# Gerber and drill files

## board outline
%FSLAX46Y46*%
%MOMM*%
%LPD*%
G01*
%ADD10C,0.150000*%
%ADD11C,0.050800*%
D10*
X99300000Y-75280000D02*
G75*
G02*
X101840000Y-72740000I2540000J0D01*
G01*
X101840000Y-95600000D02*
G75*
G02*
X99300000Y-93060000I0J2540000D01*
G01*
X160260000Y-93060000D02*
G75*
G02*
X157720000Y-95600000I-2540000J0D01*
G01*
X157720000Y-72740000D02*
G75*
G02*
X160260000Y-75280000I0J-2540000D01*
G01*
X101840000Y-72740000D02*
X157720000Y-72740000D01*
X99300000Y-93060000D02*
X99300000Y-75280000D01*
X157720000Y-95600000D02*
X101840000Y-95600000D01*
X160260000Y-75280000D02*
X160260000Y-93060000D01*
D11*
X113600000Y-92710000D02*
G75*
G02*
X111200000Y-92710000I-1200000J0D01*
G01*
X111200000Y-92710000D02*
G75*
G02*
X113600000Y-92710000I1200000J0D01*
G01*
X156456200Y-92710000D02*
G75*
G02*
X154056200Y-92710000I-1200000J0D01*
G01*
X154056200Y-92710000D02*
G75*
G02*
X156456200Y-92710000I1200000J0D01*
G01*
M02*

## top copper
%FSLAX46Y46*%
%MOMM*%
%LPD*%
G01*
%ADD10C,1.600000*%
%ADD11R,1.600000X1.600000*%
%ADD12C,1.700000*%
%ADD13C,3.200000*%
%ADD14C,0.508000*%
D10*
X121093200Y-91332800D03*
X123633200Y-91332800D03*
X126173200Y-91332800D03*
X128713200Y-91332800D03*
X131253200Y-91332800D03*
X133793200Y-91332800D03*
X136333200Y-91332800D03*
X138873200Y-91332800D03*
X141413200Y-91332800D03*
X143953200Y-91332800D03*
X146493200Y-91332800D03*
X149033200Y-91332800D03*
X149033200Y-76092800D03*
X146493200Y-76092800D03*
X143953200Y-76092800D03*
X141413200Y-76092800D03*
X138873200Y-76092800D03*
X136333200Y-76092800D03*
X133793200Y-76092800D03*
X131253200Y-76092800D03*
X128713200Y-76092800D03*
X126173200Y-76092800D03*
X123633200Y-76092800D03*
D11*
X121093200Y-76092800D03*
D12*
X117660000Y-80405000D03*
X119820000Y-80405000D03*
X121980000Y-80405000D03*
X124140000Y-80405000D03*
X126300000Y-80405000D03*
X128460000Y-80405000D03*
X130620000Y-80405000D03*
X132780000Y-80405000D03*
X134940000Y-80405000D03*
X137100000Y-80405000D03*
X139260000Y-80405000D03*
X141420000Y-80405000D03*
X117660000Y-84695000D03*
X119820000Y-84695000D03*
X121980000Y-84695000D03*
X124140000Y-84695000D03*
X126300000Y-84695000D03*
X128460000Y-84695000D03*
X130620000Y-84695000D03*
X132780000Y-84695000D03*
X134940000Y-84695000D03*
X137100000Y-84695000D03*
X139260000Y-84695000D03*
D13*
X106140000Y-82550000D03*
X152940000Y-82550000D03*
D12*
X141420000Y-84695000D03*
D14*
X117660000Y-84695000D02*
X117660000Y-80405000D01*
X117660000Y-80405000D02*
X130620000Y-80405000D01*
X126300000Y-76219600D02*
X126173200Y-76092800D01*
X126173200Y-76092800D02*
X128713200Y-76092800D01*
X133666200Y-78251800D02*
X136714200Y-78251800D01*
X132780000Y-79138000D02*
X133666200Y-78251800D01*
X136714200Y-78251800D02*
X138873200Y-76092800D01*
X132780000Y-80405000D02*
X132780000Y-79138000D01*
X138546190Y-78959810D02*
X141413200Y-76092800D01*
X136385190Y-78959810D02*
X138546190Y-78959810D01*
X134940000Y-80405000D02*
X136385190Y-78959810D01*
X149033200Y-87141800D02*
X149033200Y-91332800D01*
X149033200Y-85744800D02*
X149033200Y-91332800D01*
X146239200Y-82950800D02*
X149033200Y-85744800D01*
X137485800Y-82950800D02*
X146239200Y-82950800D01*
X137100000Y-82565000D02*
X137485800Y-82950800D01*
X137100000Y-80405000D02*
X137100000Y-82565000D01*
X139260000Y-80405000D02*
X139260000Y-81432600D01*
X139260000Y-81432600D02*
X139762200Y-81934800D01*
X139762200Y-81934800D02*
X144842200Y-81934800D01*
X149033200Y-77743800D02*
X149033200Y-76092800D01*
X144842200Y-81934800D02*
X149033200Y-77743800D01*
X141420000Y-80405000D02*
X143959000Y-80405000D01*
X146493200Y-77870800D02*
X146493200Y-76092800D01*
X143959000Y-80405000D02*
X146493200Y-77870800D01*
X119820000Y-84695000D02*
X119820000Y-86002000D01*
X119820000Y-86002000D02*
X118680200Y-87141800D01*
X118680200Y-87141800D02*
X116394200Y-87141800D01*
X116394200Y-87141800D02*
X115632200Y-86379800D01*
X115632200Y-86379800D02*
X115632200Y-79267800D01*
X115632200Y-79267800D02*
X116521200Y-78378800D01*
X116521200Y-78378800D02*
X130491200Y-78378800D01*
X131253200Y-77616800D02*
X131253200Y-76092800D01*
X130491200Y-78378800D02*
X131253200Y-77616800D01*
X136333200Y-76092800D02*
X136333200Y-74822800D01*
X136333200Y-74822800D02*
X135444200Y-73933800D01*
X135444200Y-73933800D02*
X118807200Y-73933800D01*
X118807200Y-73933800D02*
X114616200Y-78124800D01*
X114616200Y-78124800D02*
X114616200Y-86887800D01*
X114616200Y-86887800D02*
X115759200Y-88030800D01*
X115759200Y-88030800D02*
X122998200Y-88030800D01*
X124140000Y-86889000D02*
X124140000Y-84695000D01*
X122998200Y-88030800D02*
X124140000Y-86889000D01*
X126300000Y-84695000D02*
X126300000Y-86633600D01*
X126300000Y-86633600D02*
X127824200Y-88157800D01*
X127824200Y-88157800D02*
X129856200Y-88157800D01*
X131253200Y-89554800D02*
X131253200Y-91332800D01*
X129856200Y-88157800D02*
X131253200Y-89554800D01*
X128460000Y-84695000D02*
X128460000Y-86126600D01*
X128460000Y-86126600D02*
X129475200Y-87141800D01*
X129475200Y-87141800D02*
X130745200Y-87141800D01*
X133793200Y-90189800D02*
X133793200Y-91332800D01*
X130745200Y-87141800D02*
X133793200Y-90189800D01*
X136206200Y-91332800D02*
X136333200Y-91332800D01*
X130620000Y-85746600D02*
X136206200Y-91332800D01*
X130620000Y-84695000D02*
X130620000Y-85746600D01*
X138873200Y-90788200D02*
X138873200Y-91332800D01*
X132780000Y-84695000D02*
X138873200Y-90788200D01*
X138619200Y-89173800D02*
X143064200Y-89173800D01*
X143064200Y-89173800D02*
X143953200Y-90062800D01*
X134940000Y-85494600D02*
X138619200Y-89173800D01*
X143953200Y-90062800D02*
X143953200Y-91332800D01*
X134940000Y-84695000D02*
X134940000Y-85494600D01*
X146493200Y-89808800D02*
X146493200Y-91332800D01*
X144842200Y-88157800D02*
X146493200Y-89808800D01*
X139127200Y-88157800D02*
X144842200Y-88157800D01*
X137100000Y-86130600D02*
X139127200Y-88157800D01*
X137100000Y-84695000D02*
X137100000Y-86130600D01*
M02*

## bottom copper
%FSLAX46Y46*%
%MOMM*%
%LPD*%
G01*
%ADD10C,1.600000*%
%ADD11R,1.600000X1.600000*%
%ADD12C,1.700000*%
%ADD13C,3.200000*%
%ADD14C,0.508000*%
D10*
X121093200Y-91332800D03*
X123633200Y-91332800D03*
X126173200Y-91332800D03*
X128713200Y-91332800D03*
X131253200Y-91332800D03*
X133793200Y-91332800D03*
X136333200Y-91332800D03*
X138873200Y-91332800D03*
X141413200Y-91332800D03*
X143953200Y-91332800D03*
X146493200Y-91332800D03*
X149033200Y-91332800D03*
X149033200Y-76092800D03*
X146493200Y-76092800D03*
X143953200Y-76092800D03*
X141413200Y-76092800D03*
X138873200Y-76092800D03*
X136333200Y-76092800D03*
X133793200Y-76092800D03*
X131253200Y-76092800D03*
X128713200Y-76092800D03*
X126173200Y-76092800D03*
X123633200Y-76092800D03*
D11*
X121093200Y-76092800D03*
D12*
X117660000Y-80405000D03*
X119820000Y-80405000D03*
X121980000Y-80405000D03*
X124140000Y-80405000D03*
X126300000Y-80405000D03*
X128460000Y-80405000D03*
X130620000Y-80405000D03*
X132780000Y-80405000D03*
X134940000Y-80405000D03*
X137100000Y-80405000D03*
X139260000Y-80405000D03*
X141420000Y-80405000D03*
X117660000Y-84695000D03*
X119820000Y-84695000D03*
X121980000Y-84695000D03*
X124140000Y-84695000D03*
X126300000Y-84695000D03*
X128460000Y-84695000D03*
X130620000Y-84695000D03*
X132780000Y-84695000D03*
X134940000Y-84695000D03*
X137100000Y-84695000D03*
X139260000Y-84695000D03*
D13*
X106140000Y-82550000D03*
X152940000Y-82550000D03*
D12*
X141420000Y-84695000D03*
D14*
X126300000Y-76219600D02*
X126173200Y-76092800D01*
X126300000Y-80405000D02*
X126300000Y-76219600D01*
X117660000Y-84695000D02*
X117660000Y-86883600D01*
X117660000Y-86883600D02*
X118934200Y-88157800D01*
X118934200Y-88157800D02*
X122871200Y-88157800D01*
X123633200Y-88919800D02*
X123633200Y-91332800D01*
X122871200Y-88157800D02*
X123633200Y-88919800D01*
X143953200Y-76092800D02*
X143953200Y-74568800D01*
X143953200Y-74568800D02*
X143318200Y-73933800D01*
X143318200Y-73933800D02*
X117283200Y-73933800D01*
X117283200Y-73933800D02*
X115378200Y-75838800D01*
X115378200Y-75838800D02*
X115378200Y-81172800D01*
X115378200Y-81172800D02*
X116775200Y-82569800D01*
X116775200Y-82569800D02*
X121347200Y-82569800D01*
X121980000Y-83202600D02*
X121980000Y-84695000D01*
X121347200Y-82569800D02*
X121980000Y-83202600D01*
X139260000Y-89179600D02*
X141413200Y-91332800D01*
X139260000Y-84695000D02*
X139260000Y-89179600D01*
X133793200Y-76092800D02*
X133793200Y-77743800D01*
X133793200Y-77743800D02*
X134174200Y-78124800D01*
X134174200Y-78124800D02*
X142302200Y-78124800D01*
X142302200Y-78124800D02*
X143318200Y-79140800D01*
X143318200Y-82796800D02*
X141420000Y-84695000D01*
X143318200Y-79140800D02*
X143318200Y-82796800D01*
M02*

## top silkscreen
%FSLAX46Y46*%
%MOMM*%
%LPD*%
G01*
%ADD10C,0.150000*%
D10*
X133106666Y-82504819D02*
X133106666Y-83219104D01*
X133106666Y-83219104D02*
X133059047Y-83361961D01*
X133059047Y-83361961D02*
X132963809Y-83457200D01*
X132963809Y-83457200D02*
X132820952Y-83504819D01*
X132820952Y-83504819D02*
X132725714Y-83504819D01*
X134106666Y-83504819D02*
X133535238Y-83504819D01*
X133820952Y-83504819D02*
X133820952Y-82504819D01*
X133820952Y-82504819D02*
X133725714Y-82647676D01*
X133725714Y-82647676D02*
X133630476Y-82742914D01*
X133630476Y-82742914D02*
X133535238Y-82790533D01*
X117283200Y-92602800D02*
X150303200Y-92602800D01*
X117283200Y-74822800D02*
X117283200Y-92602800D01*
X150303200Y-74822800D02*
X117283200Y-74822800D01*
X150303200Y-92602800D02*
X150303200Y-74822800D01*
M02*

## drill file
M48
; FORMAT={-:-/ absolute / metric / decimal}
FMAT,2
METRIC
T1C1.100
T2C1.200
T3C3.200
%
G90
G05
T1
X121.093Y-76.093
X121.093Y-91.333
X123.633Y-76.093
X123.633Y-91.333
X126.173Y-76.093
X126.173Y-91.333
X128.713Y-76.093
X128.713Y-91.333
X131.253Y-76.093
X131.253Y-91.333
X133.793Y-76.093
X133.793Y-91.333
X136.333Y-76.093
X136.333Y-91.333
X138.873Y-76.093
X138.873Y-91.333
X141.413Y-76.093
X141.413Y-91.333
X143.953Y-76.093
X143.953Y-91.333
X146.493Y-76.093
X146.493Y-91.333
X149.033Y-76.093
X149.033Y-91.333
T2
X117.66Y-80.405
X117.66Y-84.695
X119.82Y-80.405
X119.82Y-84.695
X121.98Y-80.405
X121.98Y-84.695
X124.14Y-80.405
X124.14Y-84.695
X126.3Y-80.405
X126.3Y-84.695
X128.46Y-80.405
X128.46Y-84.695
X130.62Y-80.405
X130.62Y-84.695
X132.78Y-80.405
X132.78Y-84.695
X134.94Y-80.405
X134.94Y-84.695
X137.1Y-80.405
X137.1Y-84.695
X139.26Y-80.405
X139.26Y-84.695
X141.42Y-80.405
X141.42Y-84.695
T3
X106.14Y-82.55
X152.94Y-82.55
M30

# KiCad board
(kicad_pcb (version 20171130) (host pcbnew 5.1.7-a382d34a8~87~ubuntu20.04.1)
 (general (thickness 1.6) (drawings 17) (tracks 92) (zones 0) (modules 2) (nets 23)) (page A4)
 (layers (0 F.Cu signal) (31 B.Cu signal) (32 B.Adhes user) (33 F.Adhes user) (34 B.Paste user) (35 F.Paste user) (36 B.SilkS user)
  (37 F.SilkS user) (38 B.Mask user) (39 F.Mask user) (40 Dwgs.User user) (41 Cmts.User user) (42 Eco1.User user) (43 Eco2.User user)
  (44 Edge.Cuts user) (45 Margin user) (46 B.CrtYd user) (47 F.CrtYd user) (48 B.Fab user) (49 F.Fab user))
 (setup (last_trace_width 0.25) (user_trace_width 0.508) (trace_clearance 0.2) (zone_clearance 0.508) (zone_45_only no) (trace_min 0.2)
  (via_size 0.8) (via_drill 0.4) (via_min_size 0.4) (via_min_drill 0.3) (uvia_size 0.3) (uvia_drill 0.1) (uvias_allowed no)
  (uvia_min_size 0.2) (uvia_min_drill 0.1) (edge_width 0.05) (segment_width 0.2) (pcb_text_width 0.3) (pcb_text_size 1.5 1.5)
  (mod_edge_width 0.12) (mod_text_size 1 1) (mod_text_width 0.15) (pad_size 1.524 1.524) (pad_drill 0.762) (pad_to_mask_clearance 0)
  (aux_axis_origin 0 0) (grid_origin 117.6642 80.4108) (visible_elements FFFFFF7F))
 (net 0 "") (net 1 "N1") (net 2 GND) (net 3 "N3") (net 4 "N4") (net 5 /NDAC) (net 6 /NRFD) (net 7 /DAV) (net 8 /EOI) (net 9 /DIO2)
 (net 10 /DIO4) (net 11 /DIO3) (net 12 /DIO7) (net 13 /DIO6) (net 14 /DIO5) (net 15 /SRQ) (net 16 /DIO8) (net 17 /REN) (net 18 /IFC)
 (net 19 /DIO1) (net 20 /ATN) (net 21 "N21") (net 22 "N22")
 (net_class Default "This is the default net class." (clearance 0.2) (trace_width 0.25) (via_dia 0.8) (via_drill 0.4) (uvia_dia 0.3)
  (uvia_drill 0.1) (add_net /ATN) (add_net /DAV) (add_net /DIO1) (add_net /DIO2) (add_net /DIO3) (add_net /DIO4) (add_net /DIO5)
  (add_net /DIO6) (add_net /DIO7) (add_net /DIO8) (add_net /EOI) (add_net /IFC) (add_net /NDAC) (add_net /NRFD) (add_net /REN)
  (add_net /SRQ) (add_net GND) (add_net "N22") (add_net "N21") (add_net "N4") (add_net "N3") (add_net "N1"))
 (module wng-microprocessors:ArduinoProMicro (layer B.Cu) (at 135.0632 83.7128)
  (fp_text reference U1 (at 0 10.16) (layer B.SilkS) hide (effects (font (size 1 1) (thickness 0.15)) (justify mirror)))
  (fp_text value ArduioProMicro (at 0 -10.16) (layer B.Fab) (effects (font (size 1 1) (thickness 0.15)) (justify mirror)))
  (fp_line (start -17.78 8.89) (end 15.24 8.89) (layer F.SilkS) (width 0.15))
  (fp_line (start -17.78 -8.89) (end -17.78 8.89) (layer F.SilkS) (width 0.15))
  (fp_line (start 15.24 -8.89) (end -17.78 -8.89) (layer F.SilkS) (width 0.15))
  (fp_line (start 15.24 8.89) (end 15.24 -8.89) (layer F.SilkS) (width 0.15))
  (pad 24 thru_hole circle (at -13.97 7.62) (size 1.6 1.6) (drill 1.1) (layers *.Cu *.Mask B.SilkS) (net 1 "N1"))
  (pad 23 thru_hole circle (at -11.43 7.62) (size 1.6 1.6) (drill 1.1) (layers *.Cu *.Mask B.SilkS) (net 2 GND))
  (pad 22 thru_hole circle (at -8.89 7.62) (size 1.6 1.6) (drill 1.1) (layers *.Cu *.Mask B.SilkS) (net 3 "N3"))
  (pad 21 thru_hole circle (at -6.35 7.62) (size 1.6 1.6) (drill 1.1) (layers *.Cu *.Mask B.SilkS) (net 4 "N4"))
  (pad 20 thru_hole circle (at -3.81 7.62) (size 1.6 1.6) (drill 1.1) (layers *.Cu *.Mask B.SilkS) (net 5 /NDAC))
  (pad 19 thru_hole circle (at -1.27 7.62) (size 1.6 1.6) (drill 1.1) (layers *.Cu *.Mask B.SilkS) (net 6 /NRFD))
  (pad 18 thru_hole circle (at 1.27 7.62) (size 1.6 1.6) (drill 1.1) (layers *.Cu *.Mask B.SilkS) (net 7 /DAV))
  (pad 17 thru_hole circle (at 3.81 7.62) (size 1.6 1.6) (drill 1.1) (layers *.Cu *.Mask B.SilkS) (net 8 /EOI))
  (pad 16 thru_hole circle (at 6.35 7.62) (size 1.6 1.6) (drill 1.1) (layers *.Cu *.Mask B.SilkS) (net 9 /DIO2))
  (pad 15 thru_hole circle (at 8.89 7.62) (size 1.6 1.6) (drill 1.1) (layers *.Cu *.Mask B.SilkS) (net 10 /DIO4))
  (pad 14 thru_hole circle (at 11.43 7.62) (size 1.6 1.6) (drill 1.1) (layers *.Cu *.Mask B.SilkS) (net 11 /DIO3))
  (pad 13 thru_hole circle (at 13.97 7.62) (size 1.6 1.6) (drill 1.1) (layers *.Cu *.Mask B.SilkS) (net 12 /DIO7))
  (pad 12 thru_hole circle (at 13.97 -7.62) (size 1.6 1.6) (drill 1.1) (layers *.Cu *.Mask B.SilkS) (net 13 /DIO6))
  (pad 11 thru_hole circle (at 11.43 -7.62) (size 1.6 1.6) (drill 1.1) (layers *.Cu *.Mask B.SilkS) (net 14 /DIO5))
  (pad 10 thru_hole circle (at 8.89 -7.62) (size 1.6 1.6) (drill 1.1) (layers *.Cu *.Mask B.SilkS) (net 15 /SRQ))
  (pad 9 thru_hole circle (at 6.35 -7.62) (size 1.6 1.6) (drill 1.1) (layers *.Cu *.Mask B.SilkS) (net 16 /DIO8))
  (pad 8 thru_hole circle (at 3.81 -7.62) (size 1.6 1.6) (drill 1.1) (layers *.Cu *.Mask B.SilkS) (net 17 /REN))
  (pad 7 thru_hole circle (at 1.27 -7.62) (size 1.6 1.6) (drill 1.1) (layers *.Cu *.Mask B.SilkS) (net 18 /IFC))
  (pad 6 thru_hole circle (at -1.27 -7.62) (size 1.6 1.6) (drill 1.1) (layers *.Cu *.Mask B.SilkS) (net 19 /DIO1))
  (pad 5 thru_hole circle (at -3.81 -7.62) (size 1.6 1.6) (drill 1.1) (layers *.Cu *.Mask B.SilkS) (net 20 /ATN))
  (pad 4 thru_hole circle (at -6.35 -7.62) (size 1.6 1.6) (drill 1.1) (layers *.Cu *.Mask B.SilkS) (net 2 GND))
  (pad 3 thru_hole circle (at -8.89 -7.62) (size 1.6 1.6) (drill 1.1) (layers *.Cu *.Mask B.SilkS) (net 2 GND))
  (pad 2 thru_hole circle (at -11.43 -7.62) (size 1.6 1.6) (drill 1.1) (layers *.Cu *.Mask B.SilkS) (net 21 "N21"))
  (pad 1 thru_hole rect (at -13.97 -7.62) (size 1.6 1.6) (drill 1.1) (layers *.Cu *.Mask B.SilkS) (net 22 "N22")))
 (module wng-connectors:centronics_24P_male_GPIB (layer F.Cu) (at 129.54 82.55)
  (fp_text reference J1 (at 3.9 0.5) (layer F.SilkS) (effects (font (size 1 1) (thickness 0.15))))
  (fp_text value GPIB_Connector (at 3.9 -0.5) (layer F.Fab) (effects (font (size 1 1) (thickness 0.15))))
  (pad 24 thru_hole circle (at -11.88 -2.145) (size 1.7 1.7) (drill 1.2) (layers *.Cu *.Mask) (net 2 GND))
  (pad 23 thru_hole circle (at -9.72 -2.145) (size 1.7 1.7) (drill 1.2) (layers *.Cu *.Mask) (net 2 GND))
  (pad 22 thru_hole circle (at -7.56 -2.145) (size 1.7 1.7) (drill 1.2) (layers *.Cu *.Mask) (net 2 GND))
  (pad 21 thru_hole circle (at -5.4 -2.145) (size 1.7 1.7) (drill 1.2) (layers *.Cu *.Mask) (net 2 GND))
  (pad 20 thru_hole circle (at -3.24 -2.145) (size 1.7 1.7) (drill 1.2) (layers *.Cu *.Mask) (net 2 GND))
  (pad 19 thru_hole circle (at -1.08 -2.145) (size 1.7 1.7) (drill 1.2) (layers *.Cu *.Mask) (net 2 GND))
  (pad 18 thru_hole circle (at 1.08 -2.145) (size 1.7 1.7) (drill 1.2) (layers *.Cu *.Mask) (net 2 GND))
  (pad 17 thru_hole circle (at 3.24 -2.145) (size 1.7 1.7) (drill 1.2) (layers *.Cu *.Mask) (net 17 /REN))
  (pad 16 thru_hole circle (at 5.4 -2.145) (size 1.7 1.7) (drill 1.2) (layers *.Cu *.Mask) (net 16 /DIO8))
  (pad 15 thru_hole circle (at 7.56 -2.145) (size 1.7 1.7) (drill 1.2) (layers *.Cu *.Mask) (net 12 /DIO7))
  (pad 14 thru_hole circle (at 9.72 -2.145) (size 1.7 1.7) (drill 1.2) (layers *.Cu *.Mask) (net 13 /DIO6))
  (pad 13 thru_hole circle (at 11.88 -2.145) (size 1.7 1.7) (drill 1.2) (layers *.Cu *.Mask) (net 14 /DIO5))
  (pad 12 thru_hole circle (at -11.88 2.145) (size 1.7 1.7) (drill 1.2) (layers *.Cu *.Mask) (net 2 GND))
  (pad 11 thru_hole circle (at -9.72 2.145) (size 1.7 1.7) (drill 1.2) (layers *.Cu *.Mask) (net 20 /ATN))
  (pad 10 thru_hole circle (at -7.56 2.145) (size 1.7 1.7) (drill 1.2) (layers *.Cu *.Mask) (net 15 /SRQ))
  (pad 9 thru_hole circle (at -5.4 2.145) (size 1.7 1.7) (drill 1.2) (layers *.Cu *.Mask) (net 18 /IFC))
  (pad 8 thru_hole circle (at -3.24 2.145) (size 1.7 1.7) (drill 1.2) (layers *.Cu *.Mask) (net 5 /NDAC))
  (pad 7 thru_hole circle (at -1.08 2.145) (size 1.7 1.7) (drill 1.2) (layers *.Cu *.Mask) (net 6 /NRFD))
  (pad 6 thru_hole circle (at 1.08 2.145) (size 1.7 1.7) (drill 1.2) (layers *.Cu *.Mask) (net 7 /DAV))
  (pad 5 thru_hole circle (at 3.24 2.145) (size 1.7 1.7) (drill 1.2) (layers *.Cu *.Mask) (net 8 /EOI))
  (pad 4 thru_hole circle (at 5.4 2.145) (size 1.7 1.7) (drill 1.2) (layers *.Cu *.Mask) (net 10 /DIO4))
  (pad 3 thru_hole circle (at 7.56 2.145) (size 1.7 1.7) (drill 1.2) (layers *.Cu *.Mask) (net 11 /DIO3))
  (pad 2 thru_hole circle (at 9.72 2.145) (size 1.7 1.7) (drill 1.2) (layers *.Cu *.Mask) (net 9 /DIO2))
  (pad 26 thru_hole circle (at -23.4 0) (size 3.2 3.2) (drill 3.2) (layers *.Cu *.Mask))
  (pad 25 thru_hole circle (at 23.4 0) (size 3.2 3.2) (drill 3.2) (layers *.Cu *.Mask))
  (pad 1 thru_hole circle (at 11.88 2.145) (size 1.7 1.7) (drill 1.2) (layers *.Cu *.Mask) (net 19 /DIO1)))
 (gr_arc (start 101.84 75.28) (end 101.84 72.74) (angle -90) (layer Edge.Cuts) (width 0.15))
 (gr_arc (start 101.84 93.06) (end 99.3 93.06) (angle -90) (layer Edge.Cuts) (width 0.15))
 (gr_arc (start 157.72 93.06) (end 157.72 95.6) (angle -90) (layer Edge.Cuts) (width 0.15))
 (gr_arc (start 157.72 75.28) (end 160.26 75.28) (angle -90) (layer Edge.Cuts) (width 0.15))
 (gr_line (start 101.84 72.74) (end 157.72 72.74) (layer Edge.Cuts) (width 0.15))
 (gr_line (start 99.3 93.06) (end 99.3 75.28) (layer Edge.Cuts) (width 0.15))
 (gr_line (start 157.72 95.6) (end 101.84 95.6) (layer Edge.Cuts) (width 0.15))
 (gr_line (start 160.26 75.28) (end 160.26 93.06) (layer Edge.Cuts) (width 0.15))
 (gr_circle (center 112.4 92.71) (end 113.6 92.71) (layer Edge.Cuts) (width 0.0508))
 (gr_circle (center 155.2562 92.71) (end 156.4562 92.71) (layer Edge.Cuts) (width 0.0508))
 (segment (start 117.66 84.695) (end 117.66 80.405) (width 0.508) (layer F.Cu) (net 2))
 (segment (start 117.66 80.405) (end 130.62 80.405) (width 0.508) (layer F.Cu) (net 2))
 (segment (start 126.3 76.2196) (end 126.1732 76.0928) (width 0.508) (layer F.Cu) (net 2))
 (segment (start 126.1732 76.0928) (end 128.7132 76.0928) (width 0.508) (layer F.Cu) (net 2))
 (segment (start 126.3 76.2196) (end 126.1732 76.0928) (width 0.508) (layer B.Cu) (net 2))
 (segment (start 126.3 80.405) (end 126.3 76.2196) (width 0.508) (layer B.Cu) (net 2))
 (segment (start 117.66 84.695) (end 117.66 86.8836) (width 0.508) (layer B.Cu) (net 2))
 (segment (start 117.66 86.8836) (end 118.9342 88.1578) (width 0.508) (layer B.Cu) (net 2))
 (segment (start 118.9342 88.1578) (end 122.8712 88.1578) (width 0.508) (layer B.Cu) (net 2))
 (segment (start 123.6332 88.9198) (end 123.6332 91.3328) (width 0.508) (layer B.Cu) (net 2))
 (segment (start 122.8712 88.1578) (end 123.6332 88.9198) (width 0.508) (layer B.Cu) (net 2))
 (segment (start 133.6662 78.2518) (end 136.7142 78.2518) (width 0.508) (layer F.Cu) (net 17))
 (segment (start 132.78 79.138) (end 133.6662 78.2518) (width 0.508) (layer F.Cu) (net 17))
 (segment (start 136.7142 78.2518) (end 138.8732 76.0928) (width 0.508) (layer F.Cu) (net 17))
 (segment (start 132.78 80.405) (end 132.78 79.138) (width 0.508) (layer F.Cu) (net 17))
 (segment (start 138.54619 78.95981) (end 141.4132 76.0928) (width 0.508) (layer F.Cu) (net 16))
 (segment (start 136.38519 78.95981) (end 138.54619 78.95981) (width 0.508) (layer F.Cu) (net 16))
 (segment (start 134.94 80.405) (end 136.38519 78.95981) (width 0.508) (layer F.Cu) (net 16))
 (segment (start 149.0332 87.1418) (end 149.0332 91.3328) (width 0.508) (layer F.Cu) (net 12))
 (segment (start 149.0332 85.7448) (end 149.0332 91.3328) (width 0.508) (layer F.Cu) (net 12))
 (segment (start 146.2392 82.9508) (end 149.0332 85.7448) (width 0.508) (layer F.Cu) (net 12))
 (segment (start 137.4858 82.9508) (end 146.2392 82.9508) (width 0.508) (layer F.Cu) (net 12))
 (segment (start 137.1 82.565) (end 137.4858 82.9508) (width 0.508) (layer F.Cu) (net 12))
 (segment (start 137.1 80.405) (end 137.1 82.565) (width 0.508) (layer F.Cu) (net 12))
 (segment (start 139.26 80.405) (end 139.26 81.4326) (width 0.508) (layer F.Cu) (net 13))
 (segment (start 139.26 81.4326) (end 139.7622 81.9348) (width 0.508) (layer F.Cu) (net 13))
 (segment (start 139.7622 81.9348) (end 144.8422 81.9348) (width 0.508) (layer F.Cu) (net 13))
 (segment (start 149.0332 77.7438) (end 149.0332 76.0928) (width 0.508) (layer F.Cu) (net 13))
 (segment (start 144.8422 81.9348) (end 149.0332 77.7438) (width 0.508) (layer F.Cu) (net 13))
 (segment (start 141.42 80.405) (end 143.959 80.405) (width 0.508) (layer F.Cu) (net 14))
 (segment (start 146.4932 77.8708) (end 146.4932 76.0928) (width 0.508) (layer F.Cu) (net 14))
 (segment (start 143.959 80.405) (end 146.4932 77.8708) (width 0.508) (layer F.Cu) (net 14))
 (segment (start 119.82 84.695) (end 119.82 86.002) (width 0.508) (layer F.Cu) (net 20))
 (segment (start 119.82 86.002) (end 118.6802 87.1418) (width 0.508) (layer F.Cu) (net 20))
 (segment (start 118.6802 87.1418) (end 116.3942 87.1418) (width 0.508) (layer F.Cu) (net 20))
 (segment (start 116.3942 87.1418) (end 115.6322 86.3798) (width 0.508) (layer F.Cu) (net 20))
 (segment (start 115.6322 86.3798) (end 115.6322 79.2678) (width 0.508) (layer F.Cu) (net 20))
 (segment (start 115.6322 79.2678) (end 116.5212 78.3788) (width 0.508) (layer F.Cu) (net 20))
 (segment (start 116.5212 78.3788) (end 130.4912 78.3788) (width 0.508) (layer F.Cu) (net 20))
 (segment (start 131.2532 77.6168) (end 131.2532 76.0928) (width 0.508) (layer F.Cu) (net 20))
 (segment (start 130.4912 78.3788) (end 131.2532 77.6168) (width 0.508) (layer F.Cu) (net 20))
 (segment (start 143.9532 76.0928) (end 143.9532 74.5688) (width 0.508) (layer B.Cu) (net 15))
 (segment (start 143.9532 74.5688) (end 143.3182 73.9338) (width 0.508) (layer B.Cu) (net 15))
 (segment (start 143.3182 73.9338) (end 117.2832 73.9338) (width 0.508) (layer B.Cu) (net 15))
 (segment (start 117.2832 73.9338) (end 115.3782 75.8388) (width 0.508) (layer B.Cu) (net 15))
 (segment (start 115.3782 75.8388) (end 115.3782 81.1728) (width 0.508) (layer B.Cu) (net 15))
 (segment (start 115.3782 81.1728) (end 116.7752 82.5698) (width 0.508) (layer B.Cu) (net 15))
 (segment (start 116.7752 82.5698) (end 121.3472 82.5698) (width 0.508) (layer B.Cu) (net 15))
 (segment (start 121.98 83.2026) (end 121.98 84.695) (width 0.508) (layer B.Cu) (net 15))
 (segment (start 121.3472 82.5698) (end 121.98 83.2026) (width 0.508) (layer B.Cu) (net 15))
 (segment (start 136.3332 76.0928) (end 136.3332 74.8228) (width 0.508) (layer F.Cu) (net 18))
 (segment (start 136.3332 74.8228) (end 135.4442 73.9338) (width 0.508) (layer F.Cu) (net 18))
 (segment (start 135.4442 73.9338) (end 118.8072 73.9338) (width 0.508) (layer F.Cu) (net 18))
 (segment (start 118.8072 73.9338) (end 114.6162 78.1248) (width 0.508) (layer F.Cu) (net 18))
 (segment (start 114.6162 78.1248) (end 114.6162 86.8878) (width 0.508) (layer F.Cu) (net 18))
 (segment (start 114.6162 86.8878) (end 115.7592 88.0308) (width 0.508) (layer F.Cu) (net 18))
 (segment (start 115.7592 88.0308) (end 122.9982 88.0308) (width 0.508) (layer F.Cu) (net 18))
 (segment (start 124.14 86.889) (end 124.14 84.695) (width 0.508) (layer F.Cu) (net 18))
 (segment (start 122.9982 88.0308) (end 124.14 86.889) (width 0.508) (layer F.Cu) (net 18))
 (segment (start 126.3 84.695) (end 126.3 86.6336) (width 0.508) (layer F.Cu) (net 5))
 (segment (start 126.3 86.6336) (end 127.8242 88.1578) (width 0.508) (layer F.Cu) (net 5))
 (segment (start 127.8242 88.1578) (end 129.8562 88.1578) (width 0.508) (layer F.Cu) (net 5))
 (segment (start 131.2532 89.5548) (end 131.2532 91.3328) (width 0.508) (layer F.Cu) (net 5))
 (segment (start 129.8562 88.1578) (end 131.2532 89.5548) (width 0.508) (layer F.Cu) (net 5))
 (segment (start 128.46 84.695) (end 128.46 86.1266) (width 0.508) (layer F.Cu) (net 6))
 (segment (start 128.46 86.1266) (end 129.4752 87.1418) (width 0.508) (layer F.Cu) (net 6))
 (segment (start 129.4752 87.1418) (end 130.7452 87.1418) (width 0.508) (layer F.Cu) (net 6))
 (segment (start 133.7932 90.1898) (end 133.7932 91.3328) (width 0.508) (layer F.Cu) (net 6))
 (segment (start 130.7452 87.1418) (end 133.7932 90.1898) (width 0.508) (layer F.Cu) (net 6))
 (segment (start 136.2062 91.3328) (end 136.3332 91.3328) (width 0.508) (layer F.Cu) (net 7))
 (segment (start 130.62 85.7466) (end 136.2062 91.3328) (width 0.508) (layer F.Cu) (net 7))
 (segment (start 130.62 84.695) (end 130.62 85.7466) (width 0.508) (layer F.Cu) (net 7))
 (segment (start 138.8732 90.7882) (end 138.8732 91.3328) (width 0.508) (layer F.Cu) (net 8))
 (segment (start 132.78 84.695) (end 138.8732 90.7882) (width 0.508) (layer F.Cu) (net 8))
 (segment (start 138.6192 89.1738) (end 143.0642 89.1738) (width 0.508) (layer F.Cu) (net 10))
 (segment (start 143.0642 89.1738) (end 143.9532 90.0628) (width 0.508) (layer F.Cu) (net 10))
 (segment (start 134.94 85.4946) (end 138.6192 89.1738) (width 0.508) (layer F.Cu) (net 10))
 (segment (start 143.9532 90.0628) (end 143.9532 91.3328) (width 0.508) (layer F.Cu) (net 10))
 (segment (start 134.94 84.695) (end 134.94 85.4946) (width 0.508) (layer F.Cu) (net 10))
 (segment (start 146.4932 89.8088) (end 146.4932 91.3328) (width 0.508) (layer F.Cu) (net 11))
 (segment (start 144.8422 88.1578) (end 146.4932 89.8088) (width 0.508) (layer F.Cu) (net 11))
 (segment (start 139.1272 88.1578) (end 144.8422 88.1578) (width 0.508) (layer F.Cu) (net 11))
 (segment (start 137.1 86.1306) (end 139.1272 88.1578) (width 0.508) (layer F.Cu) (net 11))
 (segment (start 137.1 84.695) (end 137.1 86.1306) (width 0.508) (layer F.Cu) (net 11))
 (segment (start 139.26 89.1796) (end 141.4132 91.3328) (width 0.508) (layer B.Cu) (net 9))
 (segment (start 139.26 84.695) (end 139.26 89.1796) (width 0.508) (layer B.Cu) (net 9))
 (segment (start 133.7932 76.0928) (end 133.7932 77.7438) (width 0.508) (layer B.Cu) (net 19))
 (segment (start 133.7932 77.7438) (end 134.1742 78.1248) (width 0.508) (layer B.Cu) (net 19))
 (segment (start 134.1742 78.1248) (end 142.3022 78.1248) (width 0.508) (layer B.Cu) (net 19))
 (segment (start 142.3022 78.1248) (end 143.3182 79.1408) (width 0.508) (layer B.Cu) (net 19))
 (segment (start 143.3182 82.7968) (end 141.42 84.695) (width 0.508) (layer B.Cu) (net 19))
 (segment (start 143.3182 79.1408) (end 143.3182 82.7968) (width 0.508) (layer B.Cu) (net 19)))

